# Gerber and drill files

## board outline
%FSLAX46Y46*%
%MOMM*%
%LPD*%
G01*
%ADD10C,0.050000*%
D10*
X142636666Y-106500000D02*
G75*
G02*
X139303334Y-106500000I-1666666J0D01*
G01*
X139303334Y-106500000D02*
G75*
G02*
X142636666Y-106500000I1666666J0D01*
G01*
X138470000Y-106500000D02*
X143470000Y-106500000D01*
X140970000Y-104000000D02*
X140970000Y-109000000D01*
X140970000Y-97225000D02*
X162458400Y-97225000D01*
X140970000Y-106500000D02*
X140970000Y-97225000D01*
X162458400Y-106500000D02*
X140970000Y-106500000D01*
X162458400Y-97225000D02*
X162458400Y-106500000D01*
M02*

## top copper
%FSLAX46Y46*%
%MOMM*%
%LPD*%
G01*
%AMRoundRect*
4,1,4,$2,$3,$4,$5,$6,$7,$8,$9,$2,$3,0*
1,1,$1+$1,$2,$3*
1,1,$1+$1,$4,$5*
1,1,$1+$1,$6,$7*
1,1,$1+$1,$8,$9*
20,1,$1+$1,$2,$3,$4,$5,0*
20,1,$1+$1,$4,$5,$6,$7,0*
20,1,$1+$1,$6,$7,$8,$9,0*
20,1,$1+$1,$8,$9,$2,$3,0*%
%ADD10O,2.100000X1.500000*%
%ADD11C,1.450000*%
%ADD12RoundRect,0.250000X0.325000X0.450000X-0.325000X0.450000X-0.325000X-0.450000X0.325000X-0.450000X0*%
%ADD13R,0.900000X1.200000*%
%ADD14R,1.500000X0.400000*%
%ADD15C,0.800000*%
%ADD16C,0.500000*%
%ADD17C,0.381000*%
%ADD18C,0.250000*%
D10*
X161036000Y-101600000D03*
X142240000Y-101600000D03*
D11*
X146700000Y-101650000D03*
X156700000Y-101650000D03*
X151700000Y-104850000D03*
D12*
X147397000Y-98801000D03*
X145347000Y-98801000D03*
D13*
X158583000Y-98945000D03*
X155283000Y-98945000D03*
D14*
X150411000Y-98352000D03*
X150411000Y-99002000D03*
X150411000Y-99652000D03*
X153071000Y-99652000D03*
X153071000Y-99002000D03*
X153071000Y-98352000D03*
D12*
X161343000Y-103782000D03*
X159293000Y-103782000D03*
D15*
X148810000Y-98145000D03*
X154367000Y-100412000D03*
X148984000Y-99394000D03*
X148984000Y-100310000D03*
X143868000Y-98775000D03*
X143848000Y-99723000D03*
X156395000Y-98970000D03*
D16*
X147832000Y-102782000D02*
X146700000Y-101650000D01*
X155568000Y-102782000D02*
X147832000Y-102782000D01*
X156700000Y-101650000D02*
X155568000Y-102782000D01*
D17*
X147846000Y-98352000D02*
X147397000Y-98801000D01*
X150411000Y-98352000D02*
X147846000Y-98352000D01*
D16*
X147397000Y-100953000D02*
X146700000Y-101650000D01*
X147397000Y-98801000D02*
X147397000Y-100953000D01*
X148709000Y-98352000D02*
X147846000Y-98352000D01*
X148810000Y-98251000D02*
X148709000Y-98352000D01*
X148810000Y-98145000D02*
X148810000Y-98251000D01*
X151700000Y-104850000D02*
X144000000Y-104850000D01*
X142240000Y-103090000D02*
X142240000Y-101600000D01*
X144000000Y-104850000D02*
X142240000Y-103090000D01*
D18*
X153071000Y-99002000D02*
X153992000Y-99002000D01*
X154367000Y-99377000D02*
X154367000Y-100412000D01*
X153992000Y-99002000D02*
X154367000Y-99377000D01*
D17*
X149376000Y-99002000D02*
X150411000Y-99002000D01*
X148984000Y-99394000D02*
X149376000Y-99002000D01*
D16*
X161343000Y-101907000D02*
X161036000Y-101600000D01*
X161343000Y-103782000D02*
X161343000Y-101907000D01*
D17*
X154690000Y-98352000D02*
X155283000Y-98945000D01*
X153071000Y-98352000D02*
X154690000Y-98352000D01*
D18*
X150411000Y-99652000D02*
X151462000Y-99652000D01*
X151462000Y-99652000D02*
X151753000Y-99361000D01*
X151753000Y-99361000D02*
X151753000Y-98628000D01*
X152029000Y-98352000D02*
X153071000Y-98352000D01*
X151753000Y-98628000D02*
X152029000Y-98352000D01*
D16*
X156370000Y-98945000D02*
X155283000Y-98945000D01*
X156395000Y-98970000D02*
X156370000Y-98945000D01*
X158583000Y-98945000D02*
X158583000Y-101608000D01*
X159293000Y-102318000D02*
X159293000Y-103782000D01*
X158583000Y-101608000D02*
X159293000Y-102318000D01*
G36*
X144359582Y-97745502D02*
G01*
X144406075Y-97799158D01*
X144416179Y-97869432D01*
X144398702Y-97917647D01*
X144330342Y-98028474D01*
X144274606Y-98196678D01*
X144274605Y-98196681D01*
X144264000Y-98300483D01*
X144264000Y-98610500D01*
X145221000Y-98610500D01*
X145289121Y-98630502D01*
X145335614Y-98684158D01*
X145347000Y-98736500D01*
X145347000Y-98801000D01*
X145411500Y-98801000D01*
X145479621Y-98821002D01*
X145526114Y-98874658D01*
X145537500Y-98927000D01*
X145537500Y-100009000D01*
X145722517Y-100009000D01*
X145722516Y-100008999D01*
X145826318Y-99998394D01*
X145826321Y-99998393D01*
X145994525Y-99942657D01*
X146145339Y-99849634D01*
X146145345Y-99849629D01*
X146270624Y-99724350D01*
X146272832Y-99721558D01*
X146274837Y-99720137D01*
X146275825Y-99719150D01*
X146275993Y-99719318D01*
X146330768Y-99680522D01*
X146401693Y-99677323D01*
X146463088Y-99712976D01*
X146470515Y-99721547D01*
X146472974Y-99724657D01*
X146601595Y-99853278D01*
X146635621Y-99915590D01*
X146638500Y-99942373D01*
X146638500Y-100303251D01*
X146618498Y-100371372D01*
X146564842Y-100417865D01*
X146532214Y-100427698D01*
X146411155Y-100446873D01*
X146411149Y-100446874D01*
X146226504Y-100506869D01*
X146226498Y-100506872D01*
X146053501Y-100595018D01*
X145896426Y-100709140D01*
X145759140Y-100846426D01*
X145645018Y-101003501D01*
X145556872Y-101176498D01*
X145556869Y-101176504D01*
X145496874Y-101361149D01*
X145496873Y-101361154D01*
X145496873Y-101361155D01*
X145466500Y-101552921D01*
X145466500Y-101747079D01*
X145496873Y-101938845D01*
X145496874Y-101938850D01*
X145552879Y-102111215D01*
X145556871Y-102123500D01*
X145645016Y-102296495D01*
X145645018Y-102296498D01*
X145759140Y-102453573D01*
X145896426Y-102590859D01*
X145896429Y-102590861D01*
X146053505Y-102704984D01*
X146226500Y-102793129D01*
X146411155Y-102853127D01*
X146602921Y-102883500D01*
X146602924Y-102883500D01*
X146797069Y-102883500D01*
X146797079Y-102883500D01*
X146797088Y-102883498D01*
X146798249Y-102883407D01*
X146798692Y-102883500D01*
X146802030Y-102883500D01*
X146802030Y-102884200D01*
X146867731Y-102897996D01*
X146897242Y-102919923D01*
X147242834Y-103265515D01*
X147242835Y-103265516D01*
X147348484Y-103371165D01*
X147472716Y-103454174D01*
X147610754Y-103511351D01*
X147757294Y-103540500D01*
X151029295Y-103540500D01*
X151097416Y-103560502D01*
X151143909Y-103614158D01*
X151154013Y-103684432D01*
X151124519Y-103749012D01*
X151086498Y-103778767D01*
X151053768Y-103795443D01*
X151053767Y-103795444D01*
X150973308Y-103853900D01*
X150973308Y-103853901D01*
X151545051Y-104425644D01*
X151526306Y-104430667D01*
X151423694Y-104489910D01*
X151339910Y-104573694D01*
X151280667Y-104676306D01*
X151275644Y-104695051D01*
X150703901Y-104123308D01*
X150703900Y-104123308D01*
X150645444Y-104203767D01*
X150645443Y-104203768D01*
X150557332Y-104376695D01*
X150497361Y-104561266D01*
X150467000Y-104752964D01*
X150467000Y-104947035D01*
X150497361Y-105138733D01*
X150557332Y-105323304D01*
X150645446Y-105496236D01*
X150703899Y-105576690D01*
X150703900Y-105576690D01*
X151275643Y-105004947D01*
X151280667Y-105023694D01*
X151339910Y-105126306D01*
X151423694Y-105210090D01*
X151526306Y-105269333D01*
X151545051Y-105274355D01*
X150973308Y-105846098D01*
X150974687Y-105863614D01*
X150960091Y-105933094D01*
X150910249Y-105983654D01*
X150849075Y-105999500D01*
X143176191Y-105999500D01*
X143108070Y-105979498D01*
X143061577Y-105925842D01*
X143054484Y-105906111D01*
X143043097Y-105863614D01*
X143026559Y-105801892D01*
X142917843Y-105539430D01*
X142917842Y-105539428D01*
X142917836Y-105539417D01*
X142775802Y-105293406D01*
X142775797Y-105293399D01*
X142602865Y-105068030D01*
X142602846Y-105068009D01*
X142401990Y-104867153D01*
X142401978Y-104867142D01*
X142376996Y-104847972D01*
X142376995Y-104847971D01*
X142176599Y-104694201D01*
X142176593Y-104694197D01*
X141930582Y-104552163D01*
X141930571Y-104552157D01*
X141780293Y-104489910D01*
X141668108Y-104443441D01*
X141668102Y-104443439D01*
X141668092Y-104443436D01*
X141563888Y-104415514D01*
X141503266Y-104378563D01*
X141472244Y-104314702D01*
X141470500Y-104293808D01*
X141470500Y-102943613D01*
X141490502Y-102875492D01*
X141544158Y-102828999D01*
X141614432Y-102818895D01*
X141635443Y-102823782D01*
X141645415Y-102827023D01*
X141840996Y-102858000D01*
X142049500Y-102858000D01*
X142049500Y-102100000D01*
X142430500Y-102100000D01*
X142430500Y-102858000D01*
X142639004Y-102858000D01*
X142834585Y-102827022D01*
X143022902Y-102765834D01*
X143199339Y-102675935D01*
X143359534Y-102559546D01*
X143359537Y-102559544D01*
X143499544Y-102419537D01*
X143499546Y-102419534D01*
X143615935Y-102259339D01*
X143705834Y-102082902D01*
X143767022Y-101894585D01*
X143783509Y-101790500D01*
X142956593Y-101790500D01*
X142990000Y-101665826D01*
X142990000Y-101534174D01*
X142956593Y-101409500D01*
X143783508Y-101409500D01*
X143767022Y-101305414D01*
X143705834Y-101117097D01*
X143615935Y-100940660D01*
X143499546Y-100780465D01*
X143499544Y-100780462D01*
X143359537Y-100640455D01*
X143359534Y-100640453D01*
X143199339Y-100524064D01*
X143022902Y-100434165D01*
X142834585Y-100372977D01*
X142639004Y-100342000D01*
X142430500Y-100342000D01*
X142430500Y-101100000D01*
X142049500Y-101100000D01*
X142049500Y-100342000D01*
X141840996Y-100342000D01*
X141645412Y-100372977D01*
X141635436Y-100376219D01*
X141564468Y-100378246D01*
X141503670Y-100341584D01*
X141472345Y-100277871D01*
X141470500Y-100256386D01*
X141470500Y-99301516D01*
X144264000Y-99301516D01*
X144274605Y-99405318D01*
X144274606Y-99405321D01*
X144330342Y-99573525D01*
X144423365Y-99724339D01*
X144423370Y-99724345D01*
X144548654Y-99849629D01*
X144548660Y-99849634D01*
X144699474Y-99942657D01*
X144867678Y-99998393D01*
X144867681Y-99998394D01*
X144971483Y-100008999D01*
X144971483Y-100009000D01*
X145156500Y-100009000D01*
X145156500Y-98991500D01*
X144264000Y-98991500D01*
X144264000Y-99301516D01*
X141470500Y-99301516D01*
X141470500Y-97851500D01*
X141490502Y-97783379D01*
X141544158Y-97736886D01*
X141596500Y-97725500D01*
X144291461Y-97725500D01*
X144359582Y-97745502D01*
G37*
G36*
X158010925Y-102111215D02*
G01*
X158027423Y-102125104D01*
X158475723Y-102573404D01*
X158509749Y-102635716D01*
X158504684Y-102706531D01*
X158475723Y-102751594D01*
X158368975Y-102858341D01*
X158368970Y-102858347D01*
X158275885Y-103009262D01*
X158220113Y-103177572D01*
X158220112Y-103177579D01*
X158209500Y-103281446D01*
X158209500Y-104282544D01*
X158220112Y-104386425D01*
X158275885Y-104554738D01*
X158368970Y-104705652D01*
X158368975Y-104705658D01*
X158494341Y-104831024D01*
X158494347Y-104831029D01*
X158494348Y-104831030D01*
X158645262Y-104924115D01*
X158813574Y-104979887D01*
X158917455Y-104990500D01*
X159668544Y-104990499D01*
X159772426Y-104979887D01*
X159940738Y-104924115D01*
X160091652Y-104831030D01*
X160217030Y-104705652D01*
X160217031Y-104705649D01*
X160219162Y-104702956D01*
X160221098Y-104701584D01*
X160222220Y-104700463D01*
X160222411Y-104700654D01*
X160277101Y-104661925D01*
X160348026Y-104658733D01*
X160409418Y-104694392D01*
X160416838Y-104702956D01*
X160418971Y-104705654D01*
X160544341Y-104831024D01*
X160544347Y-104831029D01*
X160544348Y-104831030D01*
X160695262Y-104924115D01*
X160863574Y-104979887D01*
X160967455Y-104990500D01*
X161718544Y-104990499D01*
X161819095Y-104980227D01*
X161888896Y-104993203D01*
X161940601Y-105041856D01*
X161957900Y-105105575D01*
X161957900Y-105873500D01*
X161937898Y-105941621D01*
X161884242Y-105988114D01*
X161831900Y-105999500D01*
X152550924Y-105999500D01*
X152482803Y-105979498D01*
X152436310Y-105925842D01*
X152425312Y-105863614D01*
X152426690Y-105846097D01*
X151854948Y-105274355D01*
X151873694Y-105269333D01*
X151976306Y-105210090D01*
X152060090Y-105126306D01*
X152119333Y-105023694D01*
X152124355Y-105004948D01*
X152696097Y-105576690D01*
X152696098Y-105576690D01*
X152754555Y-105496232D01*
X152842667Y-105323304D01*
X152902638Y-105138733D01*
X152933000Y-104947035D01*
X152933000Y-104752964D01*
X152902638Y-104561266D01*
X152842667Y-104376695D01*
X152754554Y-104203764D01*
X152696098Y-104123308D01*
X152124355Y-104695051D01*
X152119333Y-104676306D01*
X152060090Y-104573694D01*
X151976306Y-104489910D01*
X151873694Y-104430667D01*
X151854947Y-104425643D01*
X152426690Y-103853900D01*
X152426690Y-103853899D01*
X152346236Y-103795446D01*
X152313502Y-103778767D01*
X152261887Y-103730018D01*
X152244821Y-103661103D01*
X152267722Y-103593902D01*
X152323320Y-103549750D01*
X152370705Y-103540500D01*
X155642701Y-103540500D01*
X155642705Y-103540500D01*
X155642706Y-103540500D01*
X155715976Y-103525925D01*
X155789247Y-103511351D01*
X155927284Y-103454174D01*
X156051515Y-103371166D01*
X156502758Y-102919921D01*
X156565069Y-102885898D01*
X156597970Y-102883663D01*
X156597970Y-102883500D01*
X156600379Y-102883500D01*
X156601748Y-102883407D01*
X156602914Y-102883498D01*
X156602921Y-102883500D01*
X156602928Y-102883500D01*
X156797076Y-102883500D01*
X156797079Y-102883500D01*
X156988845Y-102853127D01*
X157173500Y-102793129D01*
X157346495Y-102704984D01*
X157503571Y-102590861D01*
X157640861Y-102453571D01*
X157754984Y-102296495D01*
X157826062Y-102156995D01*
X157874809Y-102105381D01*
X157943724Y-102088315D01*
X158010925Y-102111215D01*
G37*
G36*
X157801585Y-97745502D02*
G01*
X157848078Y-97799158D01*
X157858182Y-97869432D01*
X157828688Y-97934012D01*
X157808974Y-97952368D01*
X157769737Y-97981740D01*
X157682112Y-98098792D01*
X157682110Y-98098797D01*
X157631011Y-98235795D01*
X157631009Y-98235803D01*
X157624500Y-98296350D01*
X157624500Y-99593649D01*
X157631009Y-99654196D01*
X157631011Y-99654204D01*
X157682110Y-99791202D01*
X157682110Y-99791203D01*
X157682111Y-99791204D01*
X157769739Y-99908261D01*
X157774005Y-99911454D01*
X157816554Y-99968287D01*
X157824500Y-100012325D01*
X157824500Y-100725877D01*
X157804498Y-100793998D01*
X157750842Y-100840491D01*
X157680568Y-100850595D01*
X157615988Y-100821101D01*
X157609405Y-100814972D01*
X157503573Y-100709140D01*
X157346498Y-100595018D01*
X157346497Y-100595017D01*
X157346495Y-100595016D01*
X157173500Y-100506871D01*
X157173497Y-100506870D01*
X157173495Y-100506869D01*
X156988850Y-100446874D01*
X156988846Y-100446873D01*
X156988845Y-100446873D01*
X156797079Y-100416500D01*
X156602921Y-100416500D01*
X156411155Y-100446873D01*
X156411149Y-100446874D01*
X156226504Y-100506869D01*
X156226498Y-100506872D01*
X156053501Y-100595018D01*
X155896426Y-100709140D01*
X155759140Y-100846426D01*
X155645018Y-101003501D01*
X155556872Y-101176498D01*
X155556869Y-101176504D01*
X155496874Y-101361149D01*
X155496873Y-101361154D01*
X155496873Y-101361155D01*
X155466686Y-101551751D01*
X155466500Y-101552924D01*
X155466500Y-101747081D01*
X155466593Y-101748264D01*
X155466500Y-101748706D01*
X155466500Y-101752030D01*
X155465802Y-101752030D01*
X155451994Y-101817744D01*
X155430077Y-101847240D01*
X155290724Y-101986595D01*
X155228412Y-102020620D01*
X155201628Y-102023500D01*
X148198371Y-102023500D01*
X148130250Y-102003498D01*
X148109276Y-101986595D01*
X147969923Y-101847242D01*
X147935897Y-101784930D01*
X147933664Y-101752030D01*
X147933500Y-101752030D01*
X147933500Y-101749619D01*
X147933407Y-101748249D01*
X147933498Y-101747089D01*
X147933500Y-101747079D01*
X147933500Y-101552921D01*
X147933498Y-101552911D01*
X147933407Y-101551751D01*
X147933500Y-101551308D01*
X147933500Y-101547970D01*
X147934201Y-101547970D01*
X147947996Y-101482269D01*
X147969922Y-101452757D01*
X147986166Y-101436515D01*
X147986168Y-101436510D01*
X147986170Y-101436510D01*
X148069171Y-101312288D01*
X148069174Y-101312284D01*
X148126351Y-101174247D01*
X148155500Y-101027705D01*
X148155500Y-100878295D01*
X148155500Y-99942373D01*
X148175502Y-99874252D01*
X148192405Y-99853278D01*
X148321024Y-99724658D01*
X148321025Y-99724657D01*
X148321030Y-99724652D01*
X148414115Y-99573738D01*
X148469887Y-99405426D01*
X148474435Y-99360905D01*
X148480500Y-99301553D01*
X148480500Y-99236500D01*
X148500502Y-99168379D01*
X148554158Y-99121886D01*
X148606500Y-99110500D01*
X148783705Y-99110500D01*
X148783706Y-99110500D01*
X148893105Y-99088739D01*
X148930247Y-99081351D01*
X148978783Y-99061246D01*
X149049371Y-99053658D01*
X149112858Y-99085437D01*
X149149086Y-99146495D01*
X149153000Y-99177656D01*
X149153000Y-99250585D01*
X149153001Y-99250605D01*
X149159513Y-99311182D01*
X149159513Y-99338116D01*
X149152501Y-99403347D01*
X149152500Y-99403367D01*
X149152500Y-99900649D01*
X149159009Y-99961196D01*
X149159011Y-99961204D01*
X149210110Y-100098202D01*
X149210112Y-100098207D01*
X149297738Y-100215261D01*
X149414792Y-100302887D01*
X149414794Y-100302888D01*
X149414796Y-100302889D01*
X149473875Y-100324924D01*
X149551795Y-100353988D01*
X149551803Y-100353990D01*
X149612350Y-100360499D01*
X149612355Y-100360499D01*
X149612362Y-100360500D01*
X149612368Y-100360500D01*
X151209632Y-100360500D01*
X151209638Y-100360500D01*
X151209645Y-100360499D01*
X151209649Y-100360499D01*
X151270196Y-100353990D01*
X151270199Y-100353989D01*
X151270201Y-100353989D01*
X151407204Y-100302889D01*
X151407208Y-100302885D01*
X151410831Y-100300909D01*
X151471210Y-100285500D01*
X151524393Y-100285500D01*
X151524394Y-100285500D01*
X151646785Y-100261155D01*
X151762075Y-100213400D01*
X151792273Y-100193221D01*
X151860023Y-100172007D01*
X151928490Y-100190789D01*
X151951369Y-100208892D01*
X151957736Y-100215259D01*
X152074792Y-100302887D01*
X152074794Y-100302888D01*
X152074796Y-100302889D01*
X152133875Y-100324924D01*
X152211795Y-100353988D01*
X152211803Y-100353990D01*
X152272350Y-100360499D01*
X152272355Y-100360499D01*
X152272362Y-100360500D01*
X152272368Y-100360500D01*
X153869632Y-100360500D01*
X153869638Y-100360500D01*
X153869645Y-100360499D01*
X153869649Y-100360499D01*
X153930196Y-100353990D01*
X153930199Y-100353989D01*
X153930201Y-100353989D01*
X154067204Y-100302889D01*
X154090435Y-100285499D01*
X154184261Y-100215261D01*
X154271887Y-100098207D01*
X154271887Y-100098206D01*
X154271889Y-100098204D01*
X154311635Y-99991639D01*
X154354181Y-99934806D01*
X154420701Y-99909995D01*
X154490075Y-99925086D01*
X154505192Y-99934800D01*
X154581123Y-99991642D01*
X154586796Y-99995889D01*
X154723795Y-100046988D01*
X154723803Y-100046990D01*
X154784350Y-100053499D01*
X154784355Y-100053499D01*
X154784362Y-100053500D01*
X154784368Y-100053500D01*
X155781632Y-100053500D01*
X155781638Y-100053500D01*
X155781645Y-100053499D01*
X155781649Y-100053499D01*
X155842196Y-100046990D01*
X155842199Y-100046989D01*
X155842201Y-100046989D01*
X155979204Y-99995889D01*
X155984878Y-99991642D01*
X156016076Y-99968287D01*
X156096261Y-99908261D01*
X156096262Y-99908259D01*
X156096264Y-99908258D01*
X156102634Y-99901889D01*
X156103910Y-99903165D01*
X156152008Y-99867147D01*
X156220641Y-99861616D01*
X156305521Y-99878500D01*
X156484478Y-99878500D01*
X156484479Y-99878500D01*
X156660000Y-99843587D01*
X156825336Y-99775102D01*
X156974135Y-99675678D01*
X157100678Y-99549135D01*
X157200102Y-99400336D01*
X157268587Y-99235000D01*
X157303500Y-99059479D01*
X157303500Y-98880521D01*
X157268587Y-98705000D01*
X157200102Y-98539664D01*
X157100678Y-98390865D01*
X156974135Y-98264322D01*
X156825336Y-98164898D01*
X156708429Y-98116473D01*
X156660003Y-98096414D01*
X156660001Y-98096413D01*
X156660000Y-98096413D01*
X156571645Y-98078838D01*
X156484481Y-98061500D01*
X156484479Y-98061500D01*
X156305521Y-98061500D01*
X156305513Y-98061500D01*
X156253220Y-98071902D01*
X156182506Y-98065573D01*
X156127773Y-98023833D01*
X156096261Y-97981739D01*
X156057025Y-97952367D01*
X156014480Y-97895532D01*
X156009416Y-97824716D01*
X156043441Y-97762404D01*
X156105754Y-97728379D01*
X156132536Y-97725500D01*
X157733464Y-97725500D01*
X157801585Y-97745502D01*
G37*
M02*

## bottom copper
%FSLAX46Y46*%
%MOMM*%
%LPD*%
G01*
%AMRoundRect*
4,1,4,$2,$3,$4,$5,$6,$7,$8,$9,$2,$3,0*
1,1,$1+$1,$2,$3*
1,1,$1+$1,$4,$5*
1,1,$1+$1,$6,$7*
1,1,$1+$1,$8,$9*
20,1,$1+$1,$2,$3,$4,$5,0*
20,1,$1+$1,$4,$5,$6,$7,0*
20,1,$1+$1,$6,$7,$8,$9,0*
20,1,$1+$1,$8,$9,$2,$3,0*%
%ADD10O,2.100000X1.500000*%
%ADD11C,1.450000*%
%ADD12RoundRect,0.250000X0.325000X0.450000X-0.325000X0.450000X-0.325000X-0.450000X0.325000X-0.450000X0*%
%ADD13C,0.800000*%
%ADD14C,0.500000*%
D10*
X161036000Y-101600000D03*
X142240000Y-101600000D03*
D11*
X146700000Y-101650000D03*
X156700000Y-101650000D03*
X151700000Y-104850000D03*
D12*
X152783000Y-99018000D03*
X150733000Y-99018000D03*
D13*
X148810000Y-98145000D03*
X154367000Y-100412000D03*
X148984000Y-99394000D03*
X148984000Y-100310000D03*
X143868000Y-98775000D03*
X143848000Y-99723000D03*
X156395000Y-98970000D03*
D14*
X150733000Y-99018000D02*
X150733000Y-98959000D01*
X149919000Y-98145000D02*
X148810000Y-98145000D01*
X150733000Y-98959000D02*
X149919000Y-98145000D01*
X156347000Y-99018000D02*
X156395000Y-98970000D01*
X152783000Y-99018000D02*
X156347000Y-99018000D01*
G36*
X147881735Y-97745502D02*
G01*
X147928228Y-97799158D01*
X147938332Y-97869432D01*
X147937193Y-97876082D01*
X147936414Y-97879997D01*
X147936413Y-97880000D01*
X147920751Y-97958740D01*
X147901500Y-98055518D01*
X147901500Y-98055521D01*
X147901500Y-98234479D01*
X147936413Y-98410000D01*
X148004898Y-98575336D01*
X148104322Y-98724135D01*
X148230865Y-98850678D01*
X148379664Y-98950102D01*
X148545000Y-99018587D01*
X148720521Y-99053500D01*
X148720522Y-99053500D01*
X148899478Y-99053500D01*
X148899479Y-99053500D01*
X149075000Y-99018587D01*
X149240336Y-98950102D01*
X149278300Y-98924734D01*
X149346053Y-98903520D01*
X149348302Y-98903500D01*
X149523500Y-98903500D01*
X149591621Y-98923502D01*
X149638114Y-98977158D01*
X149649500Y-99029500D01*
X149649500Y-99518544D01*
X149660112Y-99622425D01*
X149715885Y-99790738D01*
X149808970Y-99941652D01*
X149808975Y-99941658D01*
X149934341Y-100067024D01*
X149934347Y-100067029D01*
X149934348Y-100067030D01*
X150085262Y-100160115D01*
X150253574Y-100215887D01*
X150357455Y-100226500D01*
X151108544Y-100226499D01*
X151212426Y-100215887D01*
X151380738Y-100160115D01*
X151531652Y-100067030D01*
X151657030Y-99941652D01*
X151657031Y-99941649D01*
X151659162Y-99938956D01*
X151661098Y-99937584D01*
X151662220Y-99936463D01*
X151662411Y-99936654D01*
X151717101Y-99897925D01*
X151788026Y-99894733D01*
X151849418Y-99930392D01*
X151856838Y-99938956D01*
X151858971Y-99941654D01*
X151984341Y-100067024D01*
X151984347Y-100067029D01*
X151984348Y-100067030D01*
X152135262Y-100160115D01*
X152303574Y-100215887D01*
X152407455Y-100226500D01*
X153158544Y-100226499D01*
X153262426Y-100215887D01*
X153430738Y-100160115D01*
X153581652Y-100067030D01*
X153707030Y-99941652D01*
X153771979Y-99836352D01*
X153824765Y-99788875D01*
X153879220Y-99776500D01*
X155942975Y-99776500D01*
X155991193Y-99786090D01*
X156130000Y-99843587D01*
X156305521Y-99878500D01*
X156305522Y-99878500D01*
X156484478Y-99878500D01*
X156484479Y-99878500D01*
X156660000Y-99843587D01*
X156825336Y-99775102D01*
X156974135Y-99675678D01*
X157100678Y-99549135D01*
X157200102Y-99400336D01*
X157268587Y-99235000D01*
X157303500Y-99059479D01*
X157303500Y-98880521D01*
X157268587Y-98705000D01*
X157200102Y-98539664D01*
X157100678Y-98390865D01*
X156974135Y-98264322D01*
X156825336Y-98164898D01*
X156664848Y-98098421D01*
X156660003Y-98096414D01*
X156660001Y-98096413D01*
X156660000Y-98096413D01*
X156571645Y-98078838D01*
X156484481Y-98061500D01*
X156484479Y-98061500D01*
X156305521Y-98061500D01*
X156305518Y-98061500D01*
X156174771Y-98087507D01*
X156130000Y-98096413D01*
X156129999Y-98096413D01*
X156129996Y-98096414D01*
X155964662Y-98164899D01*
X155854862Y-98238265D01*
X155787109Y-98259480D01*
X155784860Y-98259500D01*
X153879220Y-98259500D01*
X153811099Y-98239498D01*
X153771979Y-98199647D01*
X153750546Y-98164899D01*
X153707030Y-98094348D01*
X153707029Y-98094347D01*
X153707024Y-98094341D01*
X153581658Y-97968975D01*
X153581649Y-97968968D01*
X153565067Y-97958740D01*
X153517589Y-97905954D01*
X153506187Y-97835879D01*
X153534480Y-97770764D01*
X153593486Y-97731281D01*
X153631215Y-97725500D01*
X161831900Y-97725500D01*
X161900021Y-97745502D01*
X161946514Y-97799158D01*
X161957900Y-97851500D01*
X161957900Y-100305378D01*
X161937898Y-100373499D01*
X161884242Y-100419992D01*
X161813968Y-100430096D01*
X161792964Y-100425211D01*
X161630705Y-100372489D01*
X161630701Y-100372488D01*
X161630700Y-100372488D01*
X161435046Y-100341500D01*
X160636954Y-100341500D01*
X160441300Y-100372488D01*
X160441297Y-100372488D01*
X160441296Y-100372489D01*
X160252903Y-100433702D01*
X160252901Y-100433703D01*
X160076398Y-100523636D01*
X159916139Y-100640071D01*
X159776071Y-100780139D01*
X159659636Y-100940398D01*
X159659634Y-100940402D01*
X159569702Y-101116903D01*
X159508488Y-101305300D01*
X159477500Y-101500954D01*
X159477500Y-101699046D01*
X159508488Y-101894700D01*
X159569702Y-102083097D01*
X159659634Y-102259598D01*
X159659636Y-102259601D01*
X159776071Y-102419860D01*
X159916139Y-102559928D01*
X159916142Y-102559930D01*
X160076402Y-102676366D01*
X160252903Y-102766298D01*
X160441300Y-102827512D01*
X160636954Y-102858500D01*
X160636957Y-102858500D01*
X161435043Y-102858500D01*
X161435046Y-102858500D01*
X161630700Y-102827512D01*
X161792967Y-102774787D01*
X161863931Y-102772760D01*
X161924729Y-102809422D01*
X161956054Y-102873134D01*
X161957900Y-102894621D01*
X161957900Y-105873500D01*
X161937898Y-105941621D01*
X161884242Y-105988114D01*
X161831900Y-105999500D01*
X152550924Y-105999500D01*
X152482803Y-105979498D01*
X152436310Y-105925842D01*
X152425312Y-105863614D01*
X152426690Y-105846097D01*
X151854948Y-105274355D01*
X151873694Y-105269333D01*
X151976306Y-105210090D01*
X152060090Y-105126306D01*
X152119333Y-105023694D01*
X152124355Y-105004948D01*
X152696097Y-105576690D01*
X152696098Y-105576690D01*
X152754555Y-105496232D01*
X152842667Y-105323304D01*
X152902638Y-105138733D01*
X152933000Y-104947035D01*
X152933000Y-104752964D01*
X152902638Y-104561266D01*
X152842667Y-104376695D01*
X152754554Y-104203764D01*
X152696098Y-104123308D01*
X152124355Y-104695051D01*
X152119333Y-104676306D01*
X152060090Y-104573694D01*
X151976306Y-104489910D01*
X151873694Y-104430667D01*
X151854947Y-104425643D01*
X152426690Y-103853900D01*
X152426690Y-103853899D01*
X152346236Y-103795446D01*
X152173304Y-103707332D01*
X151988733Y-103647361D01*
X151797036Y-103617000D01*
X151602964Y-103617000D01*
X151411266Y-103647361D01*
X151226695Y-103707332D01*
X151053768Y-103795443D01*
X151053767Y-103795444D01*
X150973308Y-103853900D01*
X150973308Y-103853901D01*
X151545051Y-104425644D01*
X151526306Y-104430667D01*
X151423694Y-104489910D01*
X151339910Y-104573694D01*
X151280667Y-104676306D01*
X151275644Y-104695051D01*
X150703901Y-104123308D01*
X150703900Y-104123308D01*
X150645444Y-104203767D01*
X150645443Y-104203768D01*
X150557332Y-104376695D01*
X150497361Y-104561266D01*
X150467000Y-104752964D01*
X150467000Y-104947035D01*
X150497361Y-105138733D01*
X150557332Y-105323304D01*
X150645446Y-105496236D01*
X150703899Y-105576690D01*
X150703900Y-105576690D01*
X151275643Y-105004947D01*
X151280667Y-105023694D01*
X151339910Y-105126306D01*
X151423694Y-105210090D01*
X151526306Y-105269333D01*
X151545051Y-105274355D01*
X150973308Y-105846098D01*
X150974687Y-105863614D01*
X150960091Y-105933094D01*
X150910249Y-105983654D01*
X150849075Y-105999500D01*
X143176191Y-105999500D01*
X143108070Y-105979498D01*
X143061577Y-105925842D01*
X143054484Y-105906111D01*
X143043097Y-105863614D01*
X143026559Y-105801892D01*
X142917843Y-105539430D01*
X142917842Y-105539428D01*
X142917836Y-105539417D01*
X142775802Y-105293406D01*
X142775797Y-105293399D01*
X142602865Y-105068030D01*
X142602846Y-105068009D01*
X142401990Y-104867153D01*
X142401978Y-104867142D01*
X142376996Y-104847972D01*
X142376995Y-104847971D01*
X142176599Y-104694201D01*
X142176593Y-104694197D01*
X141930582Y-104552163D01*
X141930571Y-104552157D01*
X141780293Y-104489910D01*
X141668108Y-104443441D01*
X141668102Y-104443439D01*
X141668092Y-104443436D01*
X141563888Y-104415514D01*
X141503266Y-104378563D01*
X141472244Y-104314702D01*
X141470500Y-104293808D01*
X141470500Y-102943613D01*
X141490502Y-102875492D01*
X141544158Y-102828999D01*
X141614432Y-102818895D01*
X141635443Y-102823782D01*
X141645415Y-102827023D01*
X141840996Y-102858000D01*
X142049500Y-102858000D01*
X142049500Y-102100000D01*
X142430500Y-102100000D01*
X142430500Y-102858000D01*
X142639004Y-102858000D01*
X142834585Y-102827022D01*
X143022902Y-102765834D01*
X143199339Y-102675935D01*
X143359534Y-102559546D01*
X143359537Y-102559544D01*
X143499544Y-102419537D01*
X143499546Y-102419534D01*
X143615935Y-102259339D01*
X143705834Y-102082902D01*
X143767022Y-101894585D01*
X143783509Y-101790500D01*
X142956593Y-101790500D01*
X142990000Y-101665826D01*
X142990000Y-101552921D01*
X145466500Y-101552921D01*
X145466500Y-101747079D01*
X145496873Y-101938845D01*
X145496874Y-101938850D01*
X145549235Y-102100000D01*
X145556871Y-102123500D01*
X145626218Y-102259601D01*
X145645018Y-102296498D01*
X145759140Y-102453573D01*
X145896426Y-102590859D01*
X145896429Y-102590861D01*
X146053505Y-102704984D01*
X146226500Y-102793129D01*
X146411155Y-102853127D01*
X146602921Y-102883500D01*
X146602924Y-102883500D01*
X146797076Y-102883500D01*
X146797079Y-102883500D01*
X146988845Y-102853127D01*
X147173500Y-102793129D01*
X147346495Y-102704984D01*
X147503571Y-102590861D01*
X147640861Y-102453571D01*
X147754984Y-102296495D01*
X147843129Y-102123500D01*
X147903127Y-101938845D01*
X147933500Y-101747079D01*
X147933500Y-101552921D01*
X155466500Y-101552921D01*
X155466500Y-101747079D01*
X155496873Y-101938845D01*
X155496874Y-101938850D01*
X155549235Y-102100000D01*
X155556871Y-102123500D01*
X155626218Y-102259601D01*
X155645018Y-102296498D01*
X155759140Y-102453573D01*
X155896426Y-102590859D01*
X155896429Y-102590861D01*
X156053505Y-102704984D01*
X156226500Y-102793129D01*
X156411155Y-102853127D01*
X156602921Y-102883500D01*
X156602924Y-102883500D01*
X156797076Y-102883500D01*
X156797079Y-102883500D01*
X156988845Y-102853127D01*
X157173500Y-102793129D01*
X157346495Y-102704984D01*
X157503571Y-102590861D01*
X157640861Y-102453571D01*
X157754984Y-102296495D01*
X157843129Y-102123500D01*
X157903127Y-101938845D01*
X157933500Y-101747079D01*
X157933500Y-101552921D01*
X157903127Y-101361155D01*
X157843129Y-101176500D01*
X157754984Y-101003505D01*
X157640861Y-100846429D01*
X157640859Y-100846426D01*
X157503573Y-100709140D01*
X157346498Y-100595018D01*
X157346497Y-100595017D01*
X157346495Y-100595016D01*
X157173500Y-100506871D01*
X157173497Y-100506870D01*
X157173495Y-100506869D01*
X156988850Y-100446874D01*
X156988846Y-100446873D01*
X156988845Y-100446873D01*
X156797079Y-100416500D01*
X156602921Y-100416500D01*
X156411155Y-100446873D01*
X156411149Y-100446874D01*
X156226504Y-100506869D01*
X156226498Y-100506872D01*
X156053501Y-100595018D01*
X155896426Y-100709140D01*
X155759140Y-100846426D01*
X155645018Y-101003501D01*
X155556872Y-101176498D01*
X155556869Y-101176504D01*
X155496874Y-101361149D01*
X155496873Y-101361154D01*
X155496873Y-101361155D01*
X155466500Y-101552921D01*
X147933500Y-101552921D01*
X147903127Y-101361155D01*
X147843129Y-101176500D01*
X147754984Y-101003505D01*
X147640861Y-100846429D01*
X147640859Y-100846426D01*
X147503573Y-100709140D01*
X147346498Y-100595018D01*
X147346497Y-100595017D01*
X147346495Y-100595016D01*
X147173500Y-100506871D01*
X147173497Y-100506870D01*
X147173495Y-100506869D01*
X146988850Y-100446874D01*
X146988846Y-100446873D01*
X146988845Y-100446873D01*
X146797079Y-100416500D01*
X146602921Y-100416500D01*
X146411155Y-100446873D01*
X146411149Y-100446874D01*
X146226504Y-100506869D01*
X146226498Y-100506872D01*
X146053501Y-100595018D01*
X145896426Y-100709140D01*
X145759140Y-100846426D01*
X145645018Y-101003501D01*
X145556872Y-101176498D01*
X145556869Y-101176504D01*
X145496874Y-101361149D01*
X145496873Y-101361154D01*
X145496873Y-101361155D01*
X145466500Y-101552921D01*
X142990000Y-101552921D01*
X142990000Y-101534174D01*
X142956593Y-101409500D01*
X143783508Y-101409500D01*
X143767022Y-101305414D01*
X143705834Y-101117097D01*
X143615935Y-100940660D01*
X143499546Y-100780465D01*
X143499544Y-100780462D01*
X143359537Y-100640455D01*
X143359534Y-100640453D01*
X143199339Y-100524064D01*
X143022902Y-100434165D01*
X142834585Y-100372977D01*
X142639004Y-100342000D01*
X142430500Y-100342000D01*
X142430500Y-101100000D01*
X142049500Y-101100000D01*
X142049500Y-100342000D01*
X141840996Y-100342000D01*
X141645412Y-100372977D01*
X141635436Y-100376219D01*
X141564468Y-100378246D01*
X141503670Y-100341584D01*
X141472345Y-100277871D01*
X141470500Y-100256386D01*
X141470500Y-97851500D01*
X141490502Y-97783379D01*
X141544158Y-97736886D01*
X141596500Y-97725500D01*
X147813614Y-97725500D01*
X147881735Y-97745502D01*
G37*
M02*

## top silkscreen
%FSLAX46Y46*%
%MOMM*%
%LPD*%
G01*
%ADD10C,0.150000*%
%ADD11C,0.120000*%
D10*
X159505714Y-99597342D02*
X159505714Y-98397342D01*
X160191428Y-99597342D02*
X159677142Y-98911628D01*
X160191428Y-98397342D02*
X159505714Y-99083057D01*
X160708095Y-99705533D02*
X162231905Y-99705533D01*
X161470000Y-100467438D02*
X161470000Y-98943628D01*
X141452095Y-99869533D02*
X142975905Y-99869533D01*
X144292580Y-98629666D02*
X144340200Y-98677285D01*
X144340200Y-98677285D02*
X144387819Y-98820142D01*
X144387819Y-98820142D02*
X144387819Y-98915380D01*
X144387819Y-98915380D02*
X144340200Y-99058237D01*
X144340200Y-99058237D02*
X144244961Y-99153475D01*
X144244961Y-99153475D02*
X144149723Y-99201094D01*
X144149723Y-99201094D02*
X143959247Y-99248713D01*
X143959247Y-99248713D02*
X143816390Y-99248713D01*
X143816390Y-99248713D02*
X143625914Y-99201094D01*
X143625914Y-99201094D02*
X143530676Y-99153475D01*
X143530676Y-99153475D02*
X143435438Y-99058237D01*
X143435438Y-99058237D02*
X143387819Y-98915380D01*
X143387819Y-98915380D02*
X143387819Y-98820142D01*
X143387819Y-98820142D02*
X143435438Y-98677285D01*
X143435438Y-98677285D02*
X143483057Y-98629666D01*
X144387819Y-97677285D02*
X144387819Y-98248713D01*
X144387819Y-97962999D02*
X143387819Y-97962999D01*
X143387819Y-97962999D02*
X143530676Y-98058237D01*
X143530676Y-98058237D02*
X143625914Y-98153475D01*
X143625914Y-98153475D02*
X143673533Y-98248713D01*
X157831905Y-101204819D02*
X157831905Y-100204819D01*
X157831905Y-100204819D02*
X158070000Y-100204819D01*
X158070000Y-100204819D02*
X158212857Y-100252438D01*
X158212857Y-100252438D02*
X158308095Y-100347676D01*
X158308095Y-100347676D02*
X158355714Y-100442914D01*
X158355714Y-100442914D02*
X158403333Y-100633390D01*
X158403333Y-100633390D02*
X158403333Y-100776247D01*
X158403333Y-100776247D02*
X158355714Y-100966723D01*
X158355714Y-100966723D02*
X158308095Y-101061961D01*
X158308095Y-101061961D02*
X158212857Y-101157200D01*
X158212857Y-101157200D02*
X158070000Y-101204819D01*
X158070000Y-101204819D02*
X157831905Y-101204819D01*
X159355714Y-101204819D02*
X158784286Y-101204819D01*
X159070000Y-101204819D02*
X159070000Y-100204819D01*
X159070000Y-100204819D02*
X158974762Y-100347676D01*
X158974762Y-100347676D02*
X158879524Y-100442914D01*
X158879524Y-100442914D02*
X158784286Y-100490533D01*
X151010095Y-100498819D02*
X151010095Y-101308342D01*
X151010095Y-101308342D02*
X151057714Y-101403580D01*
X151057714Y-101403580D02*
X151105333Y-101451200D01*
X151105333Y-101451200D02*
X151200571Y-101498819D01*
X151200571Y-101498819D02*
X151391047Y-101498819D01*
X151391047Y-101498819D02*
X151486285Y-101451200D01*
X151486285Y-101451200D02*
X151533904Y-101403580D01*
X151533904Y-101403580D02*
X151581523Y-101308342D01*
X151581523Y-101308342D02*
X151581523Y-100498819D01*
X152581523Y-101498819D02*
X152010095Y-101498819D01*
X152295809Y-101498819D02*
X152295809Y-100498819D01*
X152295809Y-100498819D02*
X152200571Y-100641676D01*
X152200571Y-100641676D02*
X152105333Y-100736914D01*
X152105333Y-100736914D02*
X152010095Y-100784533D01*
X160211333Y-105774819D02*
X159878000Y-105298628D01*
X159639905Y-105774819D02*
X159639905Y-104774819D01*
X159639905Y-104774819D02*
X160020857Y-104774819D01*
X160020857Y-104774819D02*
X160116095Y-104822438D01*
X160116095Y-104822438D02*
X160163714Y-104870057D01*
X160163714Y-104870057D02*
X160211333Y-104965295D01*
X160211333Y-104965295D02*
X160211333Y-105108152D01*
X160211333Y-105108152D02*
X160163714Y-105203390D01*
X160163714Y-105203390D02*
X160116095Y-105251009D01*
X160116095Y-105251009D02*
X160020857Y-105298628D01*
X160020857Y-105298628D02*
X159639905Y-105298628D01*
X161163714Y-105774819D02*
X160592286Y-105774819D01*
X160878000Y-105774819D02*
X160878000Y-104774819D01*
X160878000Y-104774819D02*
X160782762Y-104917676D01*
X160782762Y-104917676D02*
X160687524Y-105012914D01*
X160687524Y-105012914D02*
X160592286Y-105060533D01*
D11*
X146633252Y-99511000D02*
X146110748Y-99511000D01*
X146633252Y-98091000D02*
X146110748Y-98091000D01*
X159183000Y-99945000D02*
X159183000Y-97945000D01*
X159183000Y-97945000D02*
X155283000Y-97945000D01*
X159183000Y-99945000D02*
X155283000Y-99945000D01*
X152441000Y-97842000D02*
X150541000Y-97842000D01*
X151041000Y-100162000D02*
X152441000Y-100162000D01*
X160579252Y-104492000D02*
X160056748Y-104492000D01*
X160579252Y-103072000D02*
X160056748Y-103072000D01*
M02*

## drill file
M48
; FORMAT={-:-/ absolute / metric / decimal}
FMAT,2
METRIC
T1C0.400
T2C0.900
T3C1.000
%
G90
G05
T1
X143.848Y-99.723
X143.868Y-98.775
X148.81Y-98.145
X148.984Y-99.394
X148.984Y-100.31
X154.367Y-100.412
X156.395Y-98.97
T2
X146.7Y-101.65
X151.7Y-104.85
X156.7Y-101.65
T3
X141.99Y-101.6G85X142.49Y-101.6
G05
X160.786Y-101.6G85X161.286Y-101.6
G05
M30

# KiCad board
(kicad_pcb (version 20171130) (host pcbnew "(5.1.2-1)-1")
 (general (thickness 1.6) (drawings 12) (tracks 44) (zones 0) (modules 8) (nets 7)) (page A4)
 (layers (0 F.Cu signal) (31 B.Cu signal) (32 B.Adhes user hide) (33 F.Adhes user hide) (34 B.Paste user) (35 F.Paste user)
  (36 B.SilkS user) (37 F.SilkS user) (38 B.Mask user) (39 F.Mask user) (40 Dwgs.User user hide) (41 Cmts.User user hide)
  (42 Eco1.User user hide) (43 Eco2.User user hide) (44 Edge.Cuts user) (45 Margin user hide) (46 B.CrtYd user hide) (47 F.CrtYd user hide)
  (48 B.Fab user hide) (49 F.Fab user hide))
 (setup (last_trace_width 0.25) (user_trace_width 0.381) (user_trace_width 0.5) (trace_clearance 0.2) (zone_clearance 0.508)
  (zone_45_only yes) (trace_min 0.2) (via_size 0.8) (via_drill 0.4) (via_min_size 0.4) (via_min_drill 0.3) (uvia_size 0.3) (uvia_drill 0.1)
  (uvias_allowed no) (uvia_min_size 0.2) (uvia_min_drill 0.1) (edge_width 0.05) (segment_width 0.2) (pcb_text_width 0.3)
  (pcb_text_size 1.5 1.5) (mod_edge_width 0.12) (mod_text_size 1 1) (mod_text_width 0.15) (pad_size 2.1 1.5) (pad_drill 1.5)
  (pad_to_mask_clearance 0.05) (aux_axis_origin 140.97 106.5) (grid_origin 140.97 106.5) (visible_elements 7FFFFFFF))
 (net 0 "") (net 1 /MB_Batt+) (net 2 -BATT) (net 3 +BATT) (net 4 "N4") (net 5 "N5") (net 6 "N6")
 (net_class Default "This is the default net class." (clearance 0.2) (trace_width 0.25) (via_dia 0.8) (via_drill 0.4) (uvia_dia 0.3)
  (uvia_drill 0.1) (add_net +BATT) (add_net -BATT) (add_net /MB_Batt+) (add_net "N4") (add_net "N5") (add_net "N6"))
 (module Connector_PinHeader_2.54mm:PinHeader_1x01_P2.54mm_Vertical (layer B.Cu) (at 161.036 101.6)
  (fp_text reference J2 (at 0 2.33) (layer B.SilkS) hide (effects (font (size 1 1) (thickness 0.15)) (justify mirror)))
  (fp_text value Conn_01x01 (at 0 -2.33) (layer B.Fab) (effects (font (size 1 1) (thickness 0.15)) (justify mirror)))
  (pad 1 thru_hole oval (at 0 0) (size 2.1 1.5) (drill oval 1.5 1) (layers *.Cu *.Mask) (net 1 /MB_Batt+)))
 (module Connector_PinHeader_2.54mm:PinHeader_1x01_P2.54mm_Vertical (layer B.Cu) (at 142.24 101.6)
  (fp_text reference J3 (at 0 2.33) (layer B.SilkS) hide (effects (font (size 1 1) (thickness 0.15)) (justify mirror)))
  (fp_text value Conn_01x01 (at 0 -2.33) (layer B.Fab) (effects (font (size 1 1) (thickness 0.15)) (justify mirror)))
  (pad 1 thru_hole oval (at 0 0) (size 2.1 1.5) (drill oval 1.5 1) (layers *.Cu *.Mask) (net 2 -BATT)))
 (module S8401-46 (layer F.Cu) (at 151.7 103.25 180)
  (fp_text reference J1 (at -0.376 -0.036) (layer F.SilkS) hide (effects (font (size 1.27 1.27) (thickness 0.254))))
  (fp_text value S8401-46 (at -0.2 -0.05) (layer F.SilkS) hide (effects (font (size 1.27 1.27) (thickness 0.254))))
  (pad 3 thru_hole circle (at 5 1.6 180) (size 1.45 1.45) (drill 0.9) (layers *.Cu *.Mask) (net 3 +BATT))
  (pad 2 thru_hole circle (at -5 1.6 180) (size 1.45 1.45) (drill 0.9) (layers *.Cu *.Mask) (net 3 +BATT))
  (pad 1 thru_hole circle (at 0 -1.6 180) (size 1.45 1.45) (drill 0.9) (layers *.Cu *.Mask) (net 2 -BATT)))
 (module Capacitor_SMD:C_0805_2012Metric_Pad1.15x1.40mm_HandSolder (layer F.Cu) (at 146.372 98.801 180)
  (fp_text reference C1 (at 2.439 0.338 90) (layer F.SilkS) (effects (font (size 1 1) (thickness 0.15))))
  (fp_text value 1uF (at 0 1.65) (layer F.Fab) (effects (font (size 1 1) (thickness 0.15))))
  (fp_line (start -0.261252 -0.71) (end 0.261252 -0.71) (layer F.SilkS) (width 0.12))
  (fp_line (start -0.261252 0.71) (end 0.261252 0.71) (layer F.SilkS) (width 0.12))
  (pad 1 smd roundrect (at -1.025 0 180) (size 1.15 1.4) (layers F.Cu F.Paste F.Mask) (roundrect_rratio 0.217391) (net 3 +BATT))
  (pad 2 smd roundrect (at 1.025 0 180) (size 1.15 1.4) (layers F.Cu F.Paste F.Mask) (roundrect_rratio 0.217391) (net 2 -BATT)))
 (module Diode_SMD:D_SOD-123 (layer F.Cu) (at 156.933 98.945 180)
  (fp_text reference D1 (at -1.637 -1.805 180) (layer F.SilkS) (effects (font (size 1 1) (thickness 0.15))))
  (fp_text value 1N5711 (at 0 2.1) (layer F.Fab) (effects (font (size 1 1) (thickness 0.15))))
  (fp_line (start -2.25 -1) (end -2.25 1) (layer F.SilkS) (width 0.12))
  (fp_line (start -2.25 1) (end 1.65 1) (layer F.SilkS) (width 0.12))
  (fp_line (start -2.25 -1) (end 1.65 -1) (layer F.SilkS) (width 0.12))
  (pad 1 smd rect (at -1.65 0 180) (size 0.9 1.2) (layers F.Cu F.Paste F.Mask) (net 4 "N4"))
  (pad 2 smd rect (at 1.65 0 180) (size 0.9 1.2) (layers F.Cu F.Paste F.Mask) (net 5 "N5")))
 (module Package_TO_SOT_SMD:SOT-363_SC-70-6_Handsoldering (layer F.Cu) (at 151.741 99.002)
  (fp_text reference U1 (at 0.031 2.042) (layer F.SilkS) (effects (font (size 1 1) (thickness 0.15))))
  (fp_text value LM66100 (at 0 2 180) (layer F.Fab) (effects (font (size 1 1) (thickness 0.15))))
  (fp_line (start 0.7 -1.16) (end -1.2 -1.16) (layer F.SilkS) (width 0.12))
  (fp_line (start -0.7 1.16) (end 0.7 1.16) (layer F.SilkS) (width 0.12))
  (pad 1 smd rect (at -1.33 -0.65) (size 1.5 0.4) (layers F.Cu F.Paste F.Mask) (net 3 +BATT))
  (pad 2 smd rect (at -1.33 0) (size 1.5 0.4) (layers F.Cu F.Paste F.Mask) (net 2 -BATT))
  (pad 3 smd rect (at -1.33 0.65) (size 1.5 0.4) (layers F.Cu F.Paste F.Mask) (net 5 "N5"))
  (pad 4 smd rect (at 1.33 0.65) (size 1.5 0.4) (layers F.Cu F.Paste F.Mask) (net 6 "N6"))
  (pad 5 smd rect (at 1.33 0) (size 1.5 0.4) (layers F.Cu F.Paste F.Mask) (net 2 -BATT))
  (pad 6 smd rect (at 1.33 -0.65) (size 1.5 0.4) (layers F.Cu F.Paste F.Mask) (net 5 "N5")))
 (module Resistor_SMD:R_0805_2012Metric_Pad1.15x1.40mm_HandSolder (layer F.Cu) (at 160.318 103.782 180)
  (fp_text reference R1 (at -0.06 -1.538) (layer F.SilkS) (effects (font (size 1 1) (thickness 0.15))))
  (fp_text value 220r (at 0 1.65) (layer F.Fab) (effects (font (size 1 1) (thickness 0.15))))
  (fp_line (start -0.261252 -0.71) (end 0.261252 -0.71) (layer F.SilkS) (width 0.12))
  (fp_line (start -0.261252 0.71) (end 0.261252 0.71) (layer F.SilkS) (width 0.12))
  (pad 1 smd roundrect (at -1.025 0 180) (size 1.15 1.4) (layers F.Cu F.Paste F.Mask) (roundrect_rratio 0.217391) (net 1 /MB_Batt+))
  (pad 2 smd roundrect (at 1.025 0 180) (size 1.15 1.4) (layers F.Cu F.Paste F.Mask) (roundrect_rratio 0.217391) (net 4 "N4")))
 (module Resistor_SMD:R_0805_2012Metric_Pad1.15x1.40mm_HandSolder (layer B.Cu) (at 151.758 99.018 180)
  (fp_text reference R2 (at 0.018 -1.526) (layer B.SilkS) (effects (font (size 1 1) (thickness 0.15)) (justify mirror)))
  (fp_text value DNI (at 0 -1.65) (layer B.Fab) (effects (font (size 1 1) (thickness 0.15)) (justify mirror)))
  (pad 1 smd roundrect (at -1.025 0 180) (size 1.15 1.4) (layers B.Cu B.Paste B.Mask) (roundrect_rratio 0.217391) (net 5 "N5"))
  (pad 2 smd roundrect (at 1.025 0 180) (size 1.15 1.4) (layers B.Cu B.Paste B.Mask) (roundrect_rratio 0.217391) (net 3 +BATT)))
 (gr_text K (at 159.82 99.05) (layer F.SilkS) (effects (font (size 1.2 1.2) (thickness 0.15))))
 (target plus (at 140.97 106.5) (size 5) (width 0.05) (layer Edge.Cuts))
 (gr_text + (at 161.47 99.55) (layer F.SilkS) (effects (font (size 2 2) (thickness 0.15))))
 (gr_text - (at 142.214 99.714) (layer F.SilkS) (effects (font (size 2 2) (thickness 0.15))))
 (gr_line (start 140.97 97.225) (end 162.4584 97.225) (layer Edge.Cuts) (width 0.05))
 (gr_line (start 140.97 106.5) (end 140.97 97.225) (layer Edge.Cuts) (width 0.05))
 (gr_line (start 162.4584 106.5) (end 140.97 106.5) (layer Edge.Cuts) (width 0.05))
 (gr_line (start 162.4584 97.225) (end 162.4584 106.5) (layer Edge.Cuts) (width 0.05))
 (segment (start 147.832 102.782) (end 146.7 101.65) (width 0.5) (layer F.Cu) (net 3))
 (segment (start 155.568 102.782) (end 147.832 102.782) (width 0.5) (layer F.Cu) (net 3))
 (segment (start 156.7 101.65) (end 155.568 102.782) (width 0.5) (layer F.Cu) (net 3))
 (segment (start 147.846 98.352) (end 147.397 98.801) (width 0.381) (layer F.Cu) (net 3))
 (segment (start 150.411 98.352) (end 147.846 98.352) (width 0.381) (layer F.Cu) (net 3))
 (segment (start 147.397 100.953) (end 146.7 101.65) (width 0.5) (layer F.Cu) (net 3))
 (segment (start 147.397 98.801) (end 147.397 100.953) (width 0.5) (layer F.Cu) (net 3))
 (segment (start 150.733 99.018) (end 150.733 98.959) (width 0.5) (layer B.Cu) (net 3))
 (via (at 148.81 98.145) (size 0.8) (drill 0.4) (layers F.Cu B.Cu) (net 3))
 (segment (start 149.919 98.145) (end 148.81 98.145) (width 0.5) (layer B.Cu) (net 3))
 (segment (start 150.733 98.959) (end 149.919 98.145) (width 0.5) (layer B.Cu) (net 3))
 (segment (start 148.709 98.352) (end 147.846 98.352) (width 0.5) (layer F.Cu) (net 3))
 (segment (start 148.81 98.251) (end 148.709 98.352) (width 0.5) (layer F.Cu) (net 3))
 (segment (start 148.81 98.145) (end 148.81 98.251) (width 0.5) (layer F.Cu) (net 3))
 (segment (start 151.7 104.85) (end 144 104.85) (width 0.5) (layer F.Cu) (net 2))
 (segment (start 142.24 103.09) (end 142.24 101.6) (width 0.5) (layer F.Cu) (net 2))
 (segment (start 144 104.85) (end 142.24 103.09) (width 0.5) (layer F.Cu) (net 2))
 (segment (start 153.071 99.002) (end 153.992 99.002) (width 0.25) (layer F.Cu) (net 2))
 (via (at 154.367 100.412) (size 0.8) (drill 0.4) (layers F.Cu B.Cu) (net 2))
 (segment (start 154.367 99.377) (end 154.367 100.412) (width 0.25) (layer F.Cu) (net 2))
 (segment (start 153.992 99.002) (end 154.367 99.377) (width 0.25) (layer F.Cu) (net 2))
 (segment (start 149.376 99.002) (end 150.411 99.002) (width 0.381) (layer F.Cu) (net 2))
 (segment (start 148.984 99.394) (end 149.376 99.002) (width 0.381) (layer F.Cu) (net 2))
 (via (at 148.984 99.394) (size 0.8) (drill 0.4) (layers F.Cu B.Cu) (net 2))
 (via (at 148.984 100.31) (size 0.8) (drill 0.4) (layers F.Cu B.Cu) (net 2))
 (via (at 143.868 98.775) (size 0.8) (drill 0.4) (layers F.Cu B.Cu) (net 2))
 (via (at 143.848 99.723) (size 0.8) (drill 0.4) (layers F.Cu B.Cu) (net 2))
 (segment (start 161.343 101.907) (end 161.036 101.6) (width 0.5) (layer F.Cu) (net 1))
 (segment (start 161.343 103.782) (end 161.343 101.907) (width 0.5) (layer F.Cu) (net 1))
 (segment (start 154.69 98.352) (end 155.283 98.945) (width 0.381) (layer F.Cu) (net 5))
 (segment (start 153.071 98.352) (end 154.69 98.352) (width 0.381) (layer F.Cu) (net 5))
 (segment (start 150.411 99.652) (end 151.462 99.652) (width 0.25) (layer F.Cu) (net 5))
 (segment (start 151.462 99.652) (end 151.753 99.361) (width 0.25) (layer F.Cu) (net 5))
 (segment (start 151.753 99.361) (end 151.753 98.628) (width 0.25) (layer F.Cu) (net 5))
 (segment (start 152.029 98.352) (end 153.071 98.352) (width 0.25) (layer F.Cu) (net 5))
 (segment (start 151.753 98.628) (end 152.029 98.352) (width 0.25) (layer F.Cu) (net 5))
 (via (at 156.395 98.97) (size 0.8) (drill 0.4) (layers F.Cu B.Cu) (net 5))
 (segment (start 156.347 99.018) (end 156.395 98.97) (width 0.5) (layer B.Cu) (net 5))
 (segment (start 152.783 99.018) (end 156.347 99.018) (width 0.5) (layer B.Cu) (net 5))
 (segment (start 156.37 98.945) (end 155.283 98.945) (width 0.5) (layer F.Cu) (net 5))
 (segment (start 156.395 98.97) (end 156.37 98.945) (width 0.5) (layer F.Cu) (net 5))
 (segment (start 158.583 98.945) (end 158.583 101.608) (width 0.5) (layer F.Cu) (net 4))
 (segment (start 159.293 102.318) (end 159.293 103.782) (width 0.5) (layer F.Cu) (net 4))
 (segment (start 158.583 101.608) (end 159.293 102.318) (width 0.5) (layer F.Cu) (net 4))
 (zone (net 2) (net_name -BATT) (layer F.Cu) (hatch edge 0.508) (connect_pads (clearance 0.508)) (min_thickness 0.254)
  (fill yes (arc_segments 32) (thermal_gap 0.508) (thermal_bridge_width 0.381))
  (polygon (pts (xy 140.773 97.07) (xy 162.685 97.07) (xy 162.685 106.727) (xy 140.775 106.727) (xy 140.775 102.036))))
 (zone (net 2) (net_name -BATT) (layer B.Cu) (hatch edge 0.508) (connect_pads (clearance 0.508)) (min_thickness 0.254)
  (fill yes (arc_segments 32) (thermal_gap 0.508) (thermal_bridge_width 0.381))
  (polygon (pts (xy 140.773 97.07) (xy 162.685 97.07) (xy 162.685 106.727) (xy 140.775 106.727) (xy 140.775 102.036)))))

